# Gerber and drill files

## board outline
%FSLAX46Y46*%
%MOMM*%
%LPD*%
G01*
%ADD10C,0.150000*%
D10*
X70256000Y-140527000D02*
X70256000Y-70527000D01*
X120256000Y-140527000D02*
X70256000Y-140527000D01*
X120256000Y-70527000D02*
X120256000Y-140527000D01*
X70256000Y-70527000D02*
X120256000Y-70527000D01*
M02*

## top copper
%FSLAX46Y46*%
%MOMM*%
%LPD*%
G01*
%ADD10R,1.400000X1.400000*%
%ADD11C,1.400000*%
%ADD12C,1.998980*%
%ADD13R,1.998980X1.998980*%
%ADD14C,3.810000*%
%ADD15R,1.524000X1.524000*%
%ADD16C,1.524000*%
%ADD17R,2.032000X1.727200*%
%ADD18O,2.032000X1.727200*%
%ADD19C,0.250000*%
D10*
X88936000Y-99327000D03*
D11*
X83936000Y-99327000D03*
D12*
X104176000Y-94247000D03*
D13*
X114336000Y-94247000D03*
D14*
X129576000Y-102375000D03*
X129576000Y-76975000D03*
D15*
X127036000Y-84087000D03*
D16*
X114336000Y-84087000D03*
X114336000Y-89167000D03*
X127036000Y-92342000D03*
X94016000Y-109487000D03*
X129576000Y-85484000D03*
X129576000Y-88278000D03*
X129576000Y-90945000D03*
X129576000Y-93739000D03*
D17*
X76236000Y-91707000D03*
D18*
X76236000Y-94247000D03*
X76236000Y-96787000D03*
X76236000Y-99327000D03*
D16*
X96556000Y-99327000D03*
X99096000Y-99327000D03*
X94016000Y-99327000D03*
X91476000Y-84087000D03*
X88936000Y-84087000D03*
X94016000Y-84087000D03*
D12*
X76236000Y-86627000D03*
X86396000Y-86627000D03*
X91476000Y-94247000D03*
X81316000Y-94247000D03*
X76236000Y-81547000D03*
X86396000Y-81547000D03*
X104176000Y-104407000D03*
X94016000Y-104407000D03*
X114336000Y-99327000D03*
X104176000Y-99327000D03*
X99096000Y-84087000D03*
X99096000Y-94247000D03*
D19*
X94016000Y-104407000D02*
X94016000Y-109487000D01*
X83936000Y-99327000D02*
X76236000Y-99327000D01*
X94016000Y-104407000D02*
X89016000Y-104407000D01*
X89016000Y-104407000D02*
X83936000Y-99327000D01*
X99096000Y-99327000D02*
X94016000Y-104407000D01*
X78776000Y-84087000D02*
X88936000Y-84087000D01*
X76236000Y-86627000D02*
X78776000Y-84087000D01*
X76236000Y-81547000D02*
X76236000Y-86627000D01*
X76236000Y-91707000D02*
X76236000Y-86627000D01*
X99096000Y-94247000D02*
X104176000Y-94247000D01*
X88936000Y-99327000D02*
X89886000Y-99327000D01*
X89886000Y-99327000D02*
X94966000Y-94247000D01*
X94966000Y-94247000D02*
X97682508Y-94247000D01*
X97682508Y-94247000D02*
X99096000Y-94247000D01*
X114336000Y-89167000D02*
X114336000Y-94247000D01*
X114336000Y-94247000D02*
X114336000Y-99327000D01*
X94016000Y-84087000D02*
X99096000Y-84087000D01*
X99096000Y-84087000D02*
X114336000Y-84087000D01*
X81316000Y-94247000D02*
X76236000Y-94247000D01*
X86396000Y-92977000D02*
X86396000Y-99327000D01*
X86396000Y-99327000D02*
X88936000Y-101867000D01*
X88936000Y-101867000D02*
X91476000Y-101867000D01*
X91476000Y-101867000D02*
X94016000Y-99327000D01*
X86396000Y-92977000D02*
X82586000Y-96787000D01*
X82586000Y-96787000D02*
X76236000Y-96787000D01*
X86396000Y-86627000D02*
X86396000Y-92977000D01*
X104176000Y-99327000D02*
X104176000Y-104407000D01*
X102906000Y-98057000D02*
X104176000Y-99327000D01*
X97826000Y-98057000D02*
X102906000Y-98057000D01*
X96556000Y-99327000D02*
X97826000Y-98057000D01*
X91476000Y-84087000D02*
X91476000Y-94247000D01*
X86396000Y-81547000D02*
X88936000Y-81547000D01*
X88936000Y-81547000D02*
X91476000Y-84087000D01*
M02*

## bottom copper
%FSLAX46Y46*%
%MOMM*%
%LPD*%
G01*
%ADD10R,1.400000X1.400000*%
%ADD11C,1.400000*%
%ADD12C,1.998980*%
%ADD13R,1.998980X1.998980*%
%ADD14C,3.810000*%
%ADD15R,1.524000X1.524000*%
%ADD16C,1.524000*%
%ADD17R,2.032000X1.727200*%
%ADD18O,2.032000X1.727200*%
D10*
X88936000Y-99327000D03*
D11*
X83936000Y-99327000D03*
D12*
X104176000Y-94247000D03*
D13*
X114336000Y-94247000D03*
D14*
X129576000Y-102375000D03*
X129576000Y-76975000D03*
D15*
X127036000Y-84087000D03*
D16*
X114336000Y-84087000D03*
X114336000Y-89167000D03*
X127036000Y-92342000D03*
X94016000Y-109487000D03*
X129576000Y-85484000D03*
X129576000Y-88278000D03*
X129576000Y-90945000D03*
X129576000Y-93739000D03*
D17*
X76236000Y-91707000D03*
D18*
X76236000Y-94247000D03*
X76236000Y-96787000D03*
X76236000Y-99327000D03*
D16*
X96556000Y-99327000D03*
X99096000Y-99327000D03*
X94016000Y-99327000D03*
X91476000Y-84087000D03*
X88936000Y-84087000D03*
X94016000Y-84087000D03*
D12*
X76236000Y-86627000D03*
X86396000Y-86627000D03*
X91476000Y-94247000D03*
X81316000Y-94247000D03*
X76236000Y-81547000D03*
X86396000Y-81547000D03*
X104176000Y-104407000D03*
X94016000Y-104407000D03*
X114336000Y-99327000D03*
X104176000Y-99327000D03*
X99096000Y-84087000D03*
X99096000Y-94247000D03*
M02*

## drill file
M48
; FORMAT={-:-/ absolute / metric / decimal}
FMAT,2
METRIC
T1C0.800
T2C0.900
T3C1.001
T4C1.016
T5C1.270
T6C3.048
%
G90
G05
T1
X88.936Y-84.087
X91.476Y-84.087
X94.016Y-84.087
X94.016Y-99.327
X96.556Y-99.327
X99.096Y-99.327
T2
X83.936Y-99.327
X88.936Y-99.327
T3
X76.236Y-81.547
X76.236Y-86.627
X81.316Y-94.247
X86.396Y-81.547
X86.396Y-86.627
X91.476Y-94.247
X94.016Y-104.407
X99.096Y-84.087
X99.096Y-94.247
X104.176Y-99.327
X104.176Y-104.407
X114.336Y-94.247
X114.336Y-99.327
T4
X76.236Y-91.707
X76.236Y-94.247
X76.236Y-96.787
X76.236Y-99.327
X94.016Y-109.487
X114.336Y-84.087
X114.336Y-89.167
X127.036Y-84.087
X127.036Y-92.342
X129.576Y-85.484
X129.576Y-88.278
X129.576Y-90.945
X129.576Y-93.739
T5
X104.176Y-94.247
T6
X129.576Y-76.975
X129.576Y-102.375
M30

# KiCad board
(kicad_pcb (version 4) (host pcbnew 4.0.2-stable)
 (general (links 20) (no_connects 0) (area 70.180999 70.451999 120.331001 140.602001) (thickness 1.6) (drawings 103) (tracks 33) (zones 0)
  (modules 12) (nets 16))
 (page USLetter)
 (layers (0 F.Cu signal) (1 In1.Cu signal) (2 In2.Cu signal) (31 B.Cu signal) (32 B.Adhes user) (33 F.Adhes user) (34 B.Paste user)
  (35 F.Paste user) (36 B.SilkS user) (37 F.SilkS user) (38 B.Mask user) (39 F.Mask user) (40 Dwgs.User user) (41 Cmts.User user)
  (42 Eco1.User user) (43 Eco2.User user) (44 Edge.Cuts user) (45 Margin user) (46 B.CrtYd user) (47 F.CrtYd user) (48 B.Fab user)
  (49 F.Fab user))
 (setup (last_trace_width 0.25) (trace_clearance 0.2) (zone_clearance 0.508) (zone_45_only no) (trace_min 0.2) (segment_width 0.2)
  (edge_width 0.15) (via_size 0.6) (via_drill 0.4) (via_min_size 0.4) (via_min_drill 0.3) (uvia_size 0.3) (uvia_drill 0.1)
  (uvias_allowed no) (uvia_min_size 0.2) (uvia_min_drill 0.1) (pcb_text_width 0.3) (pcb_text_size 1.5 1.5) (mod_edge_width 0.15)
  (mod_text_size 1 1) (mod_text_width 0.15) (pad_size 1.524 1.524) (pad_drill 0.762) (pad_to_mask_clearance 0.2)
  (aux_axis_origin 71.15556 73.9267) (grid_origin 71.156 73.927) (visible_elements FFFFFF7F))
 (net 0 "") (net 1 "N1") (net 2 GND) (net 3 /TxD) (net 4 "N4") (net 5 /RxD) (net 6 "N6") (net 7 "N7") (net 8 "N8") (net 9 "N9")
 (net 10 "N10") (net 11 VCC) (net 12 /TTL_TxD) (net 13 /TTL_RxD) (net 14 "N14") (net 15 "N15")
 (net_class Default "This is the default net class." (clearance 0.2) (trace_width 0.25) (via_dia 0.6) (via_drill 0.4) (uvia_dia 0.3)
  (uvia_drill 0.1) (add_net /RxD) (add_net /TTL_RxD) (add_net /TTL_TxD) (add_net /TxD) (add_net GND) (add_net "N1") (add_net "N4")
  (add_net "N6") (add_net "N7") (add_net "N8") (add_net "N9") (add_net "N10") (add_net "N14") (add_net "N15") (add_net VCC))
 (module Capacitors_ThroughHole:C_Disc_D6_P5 (layer F.Cu) (at 88.936 99.327 180)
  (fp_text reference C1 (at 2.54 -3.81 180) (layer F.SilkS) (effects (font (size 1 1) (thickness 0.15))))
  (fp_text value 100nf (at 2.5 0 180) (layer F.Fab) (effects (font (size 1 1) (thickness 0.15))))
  (pad 1 thru_hole rect (at 0 0 180) (size 1.4 1.4) (drill 0.9) (layers *.Cu *.Mask F.SilkS) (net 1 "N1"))
  (pad 2 thru_hole circle (at 5 0 180) (size 1.4 1.4) (drill 0.9) (layers *.Cu *.Mask F.SilkS) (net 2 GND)))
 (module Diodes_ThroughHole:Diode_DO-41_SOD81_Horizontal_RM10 (layer F.Cu) (at 114.336 94.24446 180)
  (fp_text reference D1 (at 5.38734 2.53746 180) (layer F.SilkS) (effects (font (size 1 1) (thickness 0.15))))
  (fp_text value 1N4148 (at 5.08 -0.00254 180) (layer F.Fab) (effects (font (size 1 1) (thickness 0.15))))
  (pad 2 thru_hole circle (at 10.16 -0.00254) (size 1.99898 1.99898) (drill 1.27) (layers *.Cu *.Mask F.SilkS) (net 1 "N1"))
  (pad 1 thru_hole rect (at 0 -0.00254) (size 1.99898 1.99898) (drill 1.00076) (layers *.Cu *.Mask F.SilkS) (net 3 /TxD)))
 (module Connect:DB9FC (layer F.Cu) (at 128.306 89.548 270)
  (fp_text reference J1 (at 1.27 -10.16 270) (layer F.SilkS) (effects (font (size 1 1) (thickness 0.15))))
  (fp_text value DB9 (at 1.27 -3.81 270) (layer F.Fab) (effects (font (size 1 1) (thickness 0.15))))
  (pad "" thru_hole circle (at 12.827 -1.27 270) (size 3.81 3.81) (drill 3.048) (layers *.Cu *.Mask F.SilkS))
  (pad "" thru_hole circle (at -12.573 -1.27 270) (size 3.81 3.81) (drill 3.048) (layers *.Cu *.Mask F.SilkS))
  (pad 1 thru_hole rect (at -5.461 1.27 270) (size 1.524 1.524) (drill 1.016) (layers *.Cu *.Mask F.SilkS) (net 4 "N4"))
  (pad 2 thru_hole circle (at -5.461 13.97 270) (size 1.524 1.524) (drill 1.016) (layers *.Cu *.Mask F.SilkS) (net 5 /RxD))
  (pad 3 thru_hole circle (at -0.381 13.97 270) (size 1.524 1.524) (drill 1.016) (layers *.Cu *.Mask F.SilkS) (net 3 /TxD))
  (pad 4 thru_hole circle (at 2.794 1.27 270) (size 1.524 1.524) (drill 1.016) (layers *.Cu *.Mask F.SilkS) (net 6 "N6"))
  (pad 5 thru_hole circle (at 19.939 34.29 270) (size 1.524 1.524) (drill 1.016) (layers *.Cu *.Mask F.SilkS) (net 2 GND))
  (pad 6 thru_hole circle (at -4.064 -1.27 270) (size 1.524 1.524) (drill 1.016) (layers *.Cu *.Mask F.SilkS) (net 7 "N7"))
  (pad 7 thru_hole circle (at -1.27 -1.27 270) (size 1.524 1.524) (drill 1.016) (layers *.Cu *.Mask F.SilkS) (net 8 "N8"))
  (pad 8 thru_hole circle (at 1.397 -1.27 270) (size 1.524 1.524) (drill 1.016) (layers *.Cu *.Mask F.SilkS) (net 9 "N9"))
  (pad 9 thru_hole circle (at 4.191 -1.27 270) (size 1.524 1.524) (drill 1.016) (layers *.Cu *.Mask F.SilkS) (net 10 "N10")))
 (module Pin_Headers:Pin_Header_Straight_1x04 (layer F.Cu) (at 76.236 91.707)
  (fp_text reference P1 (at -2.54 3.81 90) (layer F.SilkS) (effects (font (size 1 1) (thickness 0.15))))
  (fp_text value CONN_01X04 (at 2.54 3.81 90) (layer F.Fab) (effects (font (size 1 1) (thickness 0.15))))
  (pad 1 thru_hole rect (at 0 0) (size 2.032 1.7272) (drill 1.016) (layers *.Cu *.Mask F.SilkS) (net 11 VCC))
  (pad 2 thru_hole oval (at 0 2.54) (size 2.032 1.7272) (drill 1.016) (layers *.Cu *.Mask F.SilkS) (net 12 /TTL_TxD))
  (pad 3 thru_hole oval (at 0 5.08) (size 2.032 1.7272) (drill 1.016) (layers *.Cu *.Mask F.SilkS) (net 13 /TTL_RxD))
  (pad 4 thru_hole oval (at 0 7.62) (size 2.032 1.7272) (drill 1.016) (layers *.Cu *.Mask F.SilkS) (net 2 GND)))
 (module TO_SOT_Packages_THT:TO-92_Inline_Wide (layer F.Cu) (at 94.016 99.327)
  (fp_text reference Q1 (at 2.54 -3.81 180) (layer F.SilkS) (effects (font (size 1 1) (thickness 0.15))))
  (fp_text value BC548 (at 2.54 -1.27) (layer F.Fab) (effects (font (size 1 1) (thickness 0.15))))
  (pad 2 thru_hole circle (at 2.54 0 90) (size 1.524 1.524) (drill 0.8) (layers *.Cu *.Mask F.SilkS) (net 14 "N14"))
  (pad 3 thru_hole circle (at 5.08 0 90) (size 1.524 1.524) (drill 0.8) (layers *.Cu *.Mask F.SilkS) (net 2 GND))
  (pad 1 thru_hole circle (at 0 0 90) (size 1.524 1.524) (drill 0.8) (layers *.Cu *.Mask F.SilkS) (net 13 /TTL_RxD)))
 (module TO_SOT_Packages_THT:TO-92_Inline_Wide (layer F.Cu) (at 94.016 84.087 180)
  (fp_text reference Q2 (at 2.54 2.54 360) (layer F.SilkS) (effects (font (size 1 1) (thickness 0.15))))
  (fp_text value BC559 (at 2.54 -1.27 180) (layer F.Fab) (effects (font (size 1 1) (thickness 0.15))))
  (pad 2 thru_hole circle (at 2.54 0 270) (size 1.524 1.524) (drill 0.8) (layers *.Cu *.Mask F.SilkS) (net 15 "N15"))
  (pad 3 thru_hole circle (at 5.08 0 270) (size 1.524 1.524) (drill 0.8) (layers *.Cu *.Mask F.SilkS) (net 11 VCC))
  (pad 1 thru_hole circle (at 0 0 270) (size 1.524 1.524) (drill 0.8) (layers *.Cu *.Mask F.SilkS) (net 5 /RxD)))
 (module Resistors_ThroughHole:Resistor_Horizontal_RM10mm (layer F.Cu) (at 76.236 86.627)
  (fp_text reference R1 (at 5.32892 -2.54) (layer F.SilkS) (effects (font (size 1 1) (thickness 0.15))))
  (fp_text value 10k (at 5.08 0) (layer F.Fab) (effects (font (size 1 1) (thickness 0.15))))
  (pad 1 thru_hole circle (at 0 0) (size 1.99898 1.99898) (drill 1.00076) (layers *.Cu *.SilkS *.Mask) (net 11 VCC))
  (pad 2 thru_hole circle (at 10.16 0) (size 1.99898 1.99898) (drill 1.00076) (layers *.Cu *.SilkS *.Mask) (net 13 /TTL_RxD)))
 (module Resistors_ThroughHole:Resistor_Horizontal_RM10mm (layer F.Cu) (at 91.476 94.247 180)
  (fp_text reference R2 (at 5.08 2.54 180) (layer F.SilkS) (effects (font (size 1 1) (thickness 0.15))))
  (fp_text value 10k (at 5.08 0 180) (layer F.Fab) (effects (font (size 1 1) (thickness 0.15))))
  (pad 1 thru_hole circle (at 0 0 180) (size 1.99898 1.99898) (drill 1.00076) (layers *.Cu *.SilkS *.Mask) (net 15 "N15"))
  (pad 2 thru_hole circle (at 10.16 0 180) (size 1.99898 1.99898) (drill 1.00076) (layers *.Cu *.SilkS *.Mask) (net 12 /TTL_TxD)))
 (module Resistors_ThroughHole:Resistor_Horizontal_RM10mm (layer F.Cu) (at 76.236 81.547)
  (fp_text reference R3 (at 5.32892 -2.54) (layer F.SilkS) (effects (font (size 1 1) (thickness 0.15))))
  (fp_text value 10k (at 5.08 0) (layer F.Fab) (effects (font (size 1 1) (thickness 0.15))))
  (pad 1 thru_hole circle (at 0 0) (size 1.99898 1.99898) (drill 1.00076) (layers *.Cu *.SilkS *.Mask) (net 11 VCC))
  (pad 2 thru_hole circle (at 10.16 0) (size 1.99898 1.99898) (drill 1.00076) (layers *.Cu *.SilkS *.Mask) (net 15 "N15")))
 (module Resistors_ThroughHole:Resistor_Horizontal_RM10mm (layer F.Cu) (at 104.176 104.407 180)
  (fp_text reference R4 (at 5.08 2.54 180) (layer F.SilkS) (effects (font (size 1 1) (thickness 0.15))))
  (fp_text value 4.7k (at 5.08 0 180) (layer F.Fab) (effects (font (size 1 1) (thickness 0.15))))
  (pad 1 thru_hole circle (at 0 0 180) (size 1.99898 1.99898) (drill 1.00076) (layers *.Cu *.SilkS *.Mask) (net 14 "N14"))
  (pad 2 thru_hole circle (at 10.16 0 180) (size 1.99898 1.99898) (drill 1.00076) (layers *.Cu *.SilkS *.Mask) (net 2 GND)))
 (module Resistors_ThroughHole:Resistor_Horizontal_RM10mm (layer F.Cu) (at 114.336 99.327 180)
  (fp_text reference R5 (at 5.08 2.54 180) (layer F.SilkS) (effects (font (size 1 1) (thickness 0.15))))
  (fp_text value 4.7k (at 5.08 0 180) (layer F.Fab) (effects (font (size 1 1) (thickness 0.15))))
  (pad 1 thru_hole circle (at 0 0 180) (size 1.99898 1.99898) (drill 1.00076) (layers *.Cu *.SilkS *.Mask) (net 3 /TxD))
  (pad 2 thru_hole circle (at 10.16 0 180) (size 1.99898 1.99898) (drill 1.00076) (layers *.Cu *.SilkS *.Mask) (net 14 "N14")))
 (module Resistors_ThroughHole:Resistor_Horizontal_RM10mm (layer F.Cu) (at 99.096 84.087 270)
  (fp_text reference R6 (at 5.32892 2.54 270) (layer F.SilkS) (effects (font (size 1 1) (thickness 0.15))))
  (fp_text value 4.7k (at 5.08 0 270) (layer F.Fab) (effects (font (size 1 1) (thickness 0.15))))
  (pad 1 thru_hole circle (at 0 0 270) (size 1.99898 1.99898) (drill 1.00076) (layers *.Cu *.SilkS *.Mask) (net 5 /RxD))
  (pad 2 thru_hole circle (at 10.16 0 270) (size 1.99898 1.99898) (drill 1.00076) (layers *.Cu *.SilkS *.Mask) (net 1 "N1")))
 (gr_line (start 70.256 140.527) (end 70.256 70.527) (angle 90) (layer Edge.Cuts) (width 0.15))
 (gr_line (start 120.256 140.527) (end 70.256 140.527) (angle 90) (layer Edge.Cuts) (width 0.15))
 (gr_line (start 120.256 70.527) (end 120.256 140.527) (angle 90) (layer Edge.Cuts) (width 0.15))
 (gr_line (start 70.256 70.527) (end 120.256 70.527) (angle 90) (layer Edge.Cuts) (width 0.15))
 (segment (start 94.016 104.407) (end 94.016 109.487) (width 0.25) (layer F.Cu) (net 2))
 (segment (start 83.936 99.327) (end 76.236 99.327) (width 0.25) (layer F.Cu) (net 2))
 (segment (start 94.016 104.407) (end 89.016 104.407) (width 0.25) (layer F.Cu) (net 2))
 (segment (start 89.016 104.407) (end 83.936 99.327) (width 0.25) (layer F.Cu) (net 2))
 (segment (start 99.096 99.327) (end 94.016 104.407) (width 0.25) (layer F.Cu) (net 2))
 (segment (start 78.776 84.087) (end 88.936 84.087) (width 0.25) (layer F.Cu) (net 11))
 (segment (start 76.236 86.627) (end 78.776 84.087) (width 0.25) (layer F.Cu) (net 11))
 (segment (start 76.236 81.547) (end 76.236 86.627) (width 0.25) (layer F.Cu) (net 11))
 (segment (start 76.236 91.707) (end 76.236 86.627) (width 0.25) (layer F.Cu) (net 11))
 (segment (start 99.096 94.247) (end 104.176 94.247) (width 0.25) (layer F.Cu) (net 1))
 (segment (start 88.936 99.327) (end 89.886 99.327) (width 0.25) (layer F.Cu) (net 1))
 (segment (start 89.886 99.327) (end 94.966 94.247) (width 0.25) (layer F.Cu) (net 1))
 (segment (start 94.966 94.247) (end 97.682508 94.247) (width 0.25) (layer F.Cu) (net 1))
 (segment (start 97.682508 94.247) (end 99.096 94.247) (width 0.25) (layer F.Cu) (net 1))
 (segment (start 114.336 89.167) (end 114.336 94.247) (width 0.25) (layer F.Cu) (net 3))
 (segment (start 114.336 94.247) (end 114.336 99.327) (width 0.25) (layer F.Cu) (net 3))
 (segment (start 94.016 84.087) (end 99.096 84.087) (width 0.25) (layer F.Cu) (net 5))
 (segment (start 99.096 84.087) (end 114.336 84.087) (width 0.25) (layer F.Cu) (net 5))
 (segment (start 81.316 94.247) (end 76.236 94.247) (width 0.25) (layer F.Cu) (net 12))
 (segment (start 86.396 92.977) (end 86.396 99.327) (width 0.25) (layer F.Cu) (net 13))
 (segment (start 86.396 99.327) (end 88.936 101.867) (width 0.25) (layer F.Cu) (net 13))
 (segment (start 88.936 101.867) (end 91.476 101.867) (width 0.25) (layer F.Cu) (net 13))
 (segment (start 91.476 101.867) (end 94.016 99.327) (width 0.25) (layer F.Cu) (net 13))
 (segment (start 86.396 92.977) (end 82.586 96.787) (width 0.25) (layer F.Cu) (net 13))
 (segment (start 82.586 96.787) (end 76.236 96.787) (width 0.25) (layer F.Cu) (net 13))
 (segment (start 86.396 86.627) (end 86.396 92.977) (width 0.25) (layer F.Cu) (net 13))
 (segment (start 104.176 99.327) (end 104.176 104.407) (width 0.25) (layer F.Cu) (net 14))
 (segment (start 102.906 98.057) (end 104.176 99.327) (width 0.25) (layer F.Cu) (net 14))
 (segment (start 97.826 98.057) (end 102.906 98.057) (width 0.25) (layer F.Cu) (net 14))
 (segment (start 96.556 99.327) (end 97.826 98.057) (width 0.25) (layer F.Cu) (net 14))
 (segment (start 91.476 84.087) (end 91.476 94.247) (width 0.25) (layer F.Cu) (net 15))
 (segment (start 86.396 81.547) (end 88.936 81.547) (width 0.25) (layer F.Cu) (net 15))
 (segment (start 88.936 81.547) (end 91.476 84.087) (width 0.25) (layer F.Cu) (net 15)))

